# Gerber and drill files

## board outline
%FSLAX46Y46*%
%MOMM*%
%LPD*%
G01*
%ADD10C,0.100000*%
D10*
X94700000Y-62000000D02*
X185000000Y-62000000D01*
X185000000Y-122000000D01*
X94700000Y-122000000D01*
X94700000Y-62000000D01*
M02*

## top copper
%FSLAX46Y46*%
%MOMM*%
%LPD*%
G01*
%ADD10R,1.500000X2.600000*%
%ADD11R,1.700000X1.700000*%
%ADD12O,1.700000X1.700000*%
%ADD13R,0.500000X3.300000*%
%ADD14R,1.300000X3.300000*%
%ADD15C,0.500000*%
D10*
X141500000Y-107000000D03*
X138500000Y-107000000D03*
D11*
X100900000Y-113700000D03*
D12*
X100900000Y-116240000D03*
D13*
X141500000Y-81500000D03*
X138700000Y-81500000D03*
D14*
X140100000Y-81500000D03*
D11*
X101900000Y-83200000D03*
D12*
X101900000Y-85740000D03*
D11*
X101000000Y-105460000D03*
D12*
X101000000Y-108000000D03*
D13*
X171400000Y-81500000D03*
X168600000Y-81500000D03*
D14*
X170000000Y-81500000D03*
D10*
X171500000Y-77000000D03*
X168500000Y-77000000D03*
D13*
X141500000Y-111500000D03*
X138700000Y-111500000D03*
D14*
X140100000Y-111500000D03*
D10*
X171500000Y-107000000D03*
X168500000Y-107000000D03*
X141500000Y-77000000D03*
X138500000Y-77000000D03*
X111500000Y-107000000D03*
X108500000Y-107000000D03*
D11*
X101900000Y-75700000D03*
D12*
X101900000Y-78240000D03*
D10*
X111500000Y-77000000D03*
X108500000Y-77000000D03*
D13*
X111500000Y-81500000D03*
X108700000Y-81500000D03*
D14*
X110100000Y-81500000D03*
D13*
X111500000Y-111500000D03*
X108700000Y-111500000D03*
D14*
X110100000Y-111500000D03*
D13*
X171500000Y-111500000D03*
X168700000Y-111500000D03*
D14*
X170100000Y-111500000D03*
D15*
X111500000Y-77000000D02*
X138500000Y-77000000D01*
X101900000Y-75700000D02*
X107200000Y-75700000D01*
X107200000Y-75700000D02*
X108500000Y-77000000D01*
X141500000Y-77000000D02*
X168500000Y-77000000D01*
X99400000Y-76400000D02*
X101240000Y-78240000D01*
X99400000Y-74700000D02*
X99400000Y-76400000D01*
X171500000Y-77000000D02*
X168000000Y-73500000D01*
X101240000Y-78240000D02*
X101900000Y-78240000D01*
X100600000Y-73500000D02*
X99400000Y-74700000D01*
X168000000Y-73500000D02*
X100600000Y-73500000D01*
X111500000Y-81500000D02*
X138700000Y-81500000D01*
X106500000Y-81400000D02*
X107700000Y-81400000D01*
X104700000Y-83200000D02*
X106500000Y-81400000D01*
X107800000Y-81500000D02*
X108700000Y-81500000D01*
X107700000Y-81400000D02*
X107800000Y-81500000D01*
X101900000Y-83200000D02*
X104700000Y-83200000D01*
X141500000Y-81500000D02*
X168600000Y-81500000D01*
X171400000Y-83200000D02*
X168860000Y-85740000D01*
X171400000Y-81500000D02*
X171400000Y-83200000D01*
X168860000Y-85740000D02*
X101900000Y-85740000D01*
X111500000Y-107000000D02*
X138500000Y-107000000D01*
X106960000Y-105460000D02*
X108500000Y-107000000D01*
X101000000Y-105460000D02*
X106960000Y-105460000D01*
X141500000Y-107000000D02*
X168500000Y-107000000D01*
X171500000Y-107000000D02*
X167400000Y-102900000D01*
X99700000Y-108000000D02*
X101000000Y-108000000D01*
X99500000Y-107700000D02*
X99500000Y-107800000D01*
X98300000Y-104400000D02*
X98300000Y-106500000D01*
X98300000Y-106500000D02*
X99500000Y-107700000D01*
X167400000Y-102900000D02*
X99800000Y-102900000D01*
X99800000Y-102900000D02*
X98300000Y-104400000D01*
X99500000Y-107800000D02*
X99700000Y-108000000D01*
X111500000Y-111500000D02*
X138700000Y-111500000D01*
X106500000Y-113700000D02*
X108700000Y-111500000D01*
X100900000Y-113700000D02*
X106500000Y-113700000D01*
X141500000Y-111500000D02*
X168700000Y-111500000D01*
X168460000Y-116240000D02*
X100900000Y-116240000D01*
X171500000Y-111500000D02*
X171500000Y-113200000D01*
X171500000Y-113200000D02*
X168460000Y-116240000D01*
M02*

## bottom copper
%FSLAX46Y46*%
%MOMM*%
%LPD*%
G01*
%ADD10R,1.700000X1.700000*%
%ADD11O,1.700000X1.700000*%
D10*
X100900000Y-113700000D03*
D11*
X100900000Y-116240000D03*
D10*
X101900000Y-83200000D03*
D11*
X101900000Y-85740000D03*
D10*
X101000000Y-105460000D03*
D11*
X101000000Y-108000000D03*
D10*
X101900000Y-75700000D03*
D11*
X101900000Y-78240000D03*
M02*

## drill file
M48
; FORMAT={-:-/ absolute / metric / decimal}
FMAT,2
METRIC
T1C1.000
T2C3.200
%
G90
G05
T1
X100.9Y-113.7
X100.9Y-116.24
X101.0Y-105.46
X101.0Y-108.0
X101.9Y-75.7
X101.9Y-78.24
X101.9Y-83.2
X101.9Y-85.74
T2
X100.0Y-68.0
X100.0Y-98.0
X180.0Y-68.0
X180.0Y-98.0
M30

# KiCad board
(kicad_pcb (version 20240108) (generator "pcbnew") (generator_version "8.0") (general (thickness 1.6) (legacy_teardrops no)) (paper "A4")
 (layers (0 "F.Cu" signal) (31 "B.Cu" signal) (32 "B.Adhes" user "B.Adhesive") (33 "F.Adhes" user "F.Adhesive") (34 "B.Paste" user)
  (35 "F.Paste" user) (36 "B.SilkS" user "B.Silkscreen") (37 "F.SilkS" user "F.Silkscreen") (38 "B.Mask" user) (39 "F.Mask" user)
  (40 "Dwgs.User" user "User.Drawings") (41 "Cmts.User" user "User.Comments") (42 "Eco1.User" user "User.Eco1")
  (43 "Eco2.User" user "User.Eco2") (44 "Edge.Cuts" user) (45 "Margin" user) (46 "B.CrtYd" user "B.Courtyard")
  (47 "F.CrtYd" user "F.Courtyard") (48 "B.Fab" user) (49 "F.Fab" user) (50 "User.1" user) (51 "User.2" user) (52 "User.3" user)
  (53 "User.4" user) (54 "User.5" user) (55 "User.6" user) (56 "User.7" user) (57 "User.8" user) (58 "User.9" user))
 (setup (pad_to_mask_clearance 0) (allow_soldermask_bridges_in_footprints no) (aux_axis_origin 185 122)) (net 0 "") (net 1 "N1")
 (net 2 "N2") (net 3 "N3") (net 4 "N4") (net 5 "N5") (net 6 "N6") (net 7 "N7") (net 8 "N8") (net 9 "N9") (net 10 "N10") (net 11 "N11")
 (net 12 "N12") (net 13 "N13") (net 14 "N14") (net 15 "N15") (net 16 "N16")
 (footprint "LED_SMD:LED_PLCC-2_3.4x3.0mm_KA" (layer "F.Cu") (at 140 107 180)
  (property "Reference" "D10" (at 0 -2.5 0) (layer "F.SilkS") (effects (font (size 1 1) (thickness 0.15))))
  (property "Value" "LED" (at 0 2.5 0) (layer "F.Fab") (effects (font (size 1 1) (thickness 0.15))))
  (pad "1" smd rect (at -1.5 0 180) (size 1.5 2.6) (layers "F.Cu" "F.Paste" "F.Mask") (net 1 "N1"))
  (pad "2" smd rect (at 1.5 0 180) (size 1.5 2.6) (layers "F.Cu" "F.Paste" "F.Mask") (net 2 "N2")))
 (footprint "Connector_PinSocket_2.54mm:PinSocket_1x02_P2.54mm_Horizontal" (layer "F.Cu") (at 100.9 113.7)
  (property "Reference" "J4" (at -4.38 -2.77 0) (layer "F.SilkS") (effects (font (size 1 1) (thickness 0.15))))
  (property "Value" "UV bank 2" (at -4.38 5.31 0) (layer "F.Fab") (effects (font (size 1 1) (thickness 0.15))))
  (pad "1" thru_hole rect (at 0 0) (size 1.7 1.7) (drill 1) (layers "*.Cu" "*.Mask") (remove_unused_layers no) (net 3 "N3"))
  (pad "2" thru_hole oval (at 0 2.54) (size 1.7 1.7) (drill 1) (layers "*.Cu" "*.Mask") (remove_unused_layers no) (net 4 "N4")))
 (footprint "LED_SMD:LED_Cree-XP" (layer "F.Cu") (at 140.1 81.5 180)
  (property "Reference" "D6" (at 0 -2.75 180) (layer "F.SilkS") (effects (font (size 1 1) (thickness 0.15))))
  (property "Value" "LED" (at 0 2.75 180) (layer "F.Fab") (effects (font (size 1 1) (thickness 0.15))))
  (pad "" smd rect (at 0 -1 180) (size 1.01 0.75) (layers "F.Paste"))
  (pad "" smd rect (at 0 0 180) (size 1.01 0.75) (layers "F.Paste"))
  (pad "" smd rect (at 0 1 180) (size 1.01 0.75) (layers "F.Paste"))
  (pad "1" smd rect (at -1.4 0 180) (size 0.5 3.3) (layers "F.Cu" "F.Paste" "F.Mask") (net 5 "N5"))
  (pad "2" smd rect (at 1.4 0 180) (size 0.5 3.3) (layers "F.Cu" "F.Paste" "F.Mask") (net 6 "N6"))
  (pad "3" smd rect (at 0 0 180) (size 1.3 3.3) (layers "F.Cu" "F.Mask")))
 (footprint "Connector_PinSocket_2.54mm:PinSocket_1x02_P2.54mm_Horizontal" (layer "F.Cu") (at 101.9 83.2)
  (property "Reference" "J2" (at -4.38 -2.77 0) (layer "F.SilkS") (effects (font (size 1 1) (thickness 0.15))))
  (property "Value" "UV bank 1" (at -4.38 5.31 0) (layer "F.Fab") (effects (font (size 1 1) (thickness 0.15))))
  (pad "1" thru_hole rect (at 0 0) (size 1.7 1.7) (drill 1) (layers "*.Cu" "*.Mask") (remove_unused_layers no) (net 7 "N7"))
  (pad "2" thru_hole oval (at 0 2.54) (size 1.7 1.7) (drill 1) (layers "*.Cu" "*.Mask") (remove_unused_layers no) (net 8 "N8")))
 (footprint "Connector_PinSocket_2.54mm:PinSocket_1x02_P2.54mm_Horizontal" (layer "F.Cu") (at 101 105.46)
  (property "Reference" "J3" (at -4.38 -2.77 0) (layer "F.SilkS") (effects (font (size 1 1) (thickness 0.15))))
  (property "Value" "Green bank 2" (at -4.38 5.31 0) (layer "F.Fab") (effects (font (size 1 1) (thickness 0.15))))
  (pad "1" thru_hole rect (at 0 0) (size 1.7 1.7) (drill 1) (layers "*.Cu" "*.Mask") (remove_unused_layers no) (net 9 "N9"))
  (pad "2" thru_hole oval (at 0 2.54) (size 1.7 1.7) (drill 1) (layers "*.Cu" "*.Mask") (remove_unused_layers no) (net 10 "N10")))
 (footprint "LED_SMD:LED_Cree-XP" (layer "F.Cu") (at 170 81.5 180)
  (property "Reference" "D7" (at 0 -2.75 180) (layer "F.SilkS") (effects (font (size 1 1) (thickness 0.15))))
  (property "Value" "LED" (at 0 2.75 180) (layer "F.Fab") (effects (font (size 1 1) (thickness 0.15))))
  (pad "" smd rect (at 0 -1 180) (size 1.01 0.75) (layers "F.Paste"))
  (pad "" smd rect (at 0 0 180) (size 1.01 0.75) (layers "F.Paste"))
  (pad "" smd rect (at 0 1 180) (size 1.01 0.75) (layers "F.Paste"))
  (pad "1" smd rect (at -1.4 0 180) (size 0.5 3.3) (layers "F.Cu" "F.Paste" "F.Mask") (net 8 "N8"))
  (pad "2" smd rect (at 1.4 0 180) (size 0.5 3.3) (layers "F.Cu" "F.Paste" "F.Mask") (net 5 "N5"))
  (pad "3" smd rect (at 0 0 180) (size 1.3 3.3) (layers "F.Cu" "F.Mask")))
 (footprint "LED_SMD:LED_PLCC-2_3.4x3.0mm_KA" (layer "F.Cu") (at 170 77 180)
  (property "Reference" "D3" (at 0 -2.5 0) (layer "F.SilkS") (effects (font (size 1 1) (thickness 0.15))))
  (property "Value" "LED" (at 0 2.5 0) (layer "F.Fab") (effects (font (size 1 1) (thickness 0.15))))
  (pad "1" smd rect (at -1.5 0 180) (size 1.5 2.6) (layers "F.Cu" "F.Paste" "F.Mask") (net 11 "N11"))
  (pad "2" smd rect (at 1.5 0 180) (size 1.5 2.6) (layers "F.Cu" "F.Paste" "F.Mask") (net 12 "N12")))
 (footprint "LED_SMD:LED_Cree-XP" (layer "F.Cu") (at 140.1 111.5 180)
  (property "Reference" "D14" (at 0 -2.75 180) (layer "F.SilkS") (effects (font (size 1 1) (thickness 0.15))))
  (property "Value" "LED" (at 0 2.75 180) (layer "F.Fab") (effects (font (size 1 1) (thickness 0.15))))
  (pad "" smd rect (at 0 -1 180) (size 1.01 0.75) (layers "F.Paste"))
  (pad "" smd rect (at 0 0 180) (size 1.01 0.75) (layers "F.Paste"))
  (pad "" smd rect (at 0 1 180) (size 1.01 0.75) (layers "F.Paste"))
  (pad "1" smd rect (at -1.4 0 180) (size 0.5 3.3) (layers "F.Cu" "F.Paste" "F.Mask") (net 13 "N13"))
  (pad "2" smd rect (at 1.4 0 180) (size 0.5 3.3) (layers "F.Cu" "F.Paste" "F.Mask") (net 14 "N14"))
  (pad "3" smd rect (at 0 0 180) (size 1.3 3.3) (layers "F.Cu" "F.Mask")))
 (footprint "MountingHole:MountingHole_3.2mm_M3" (layer "F.Cu") (at 180 68)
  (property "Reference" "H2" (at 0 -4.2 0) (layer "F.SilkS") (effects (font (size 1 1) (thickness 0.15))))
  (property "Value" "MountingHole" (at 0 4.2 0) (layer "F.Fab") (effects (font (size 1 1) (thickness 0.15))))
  (pad "" np_thru_hole circle (at 0 0) (size 3.2 3.2) (drill 3.2) (layers "*.Cu" "*.Mask")))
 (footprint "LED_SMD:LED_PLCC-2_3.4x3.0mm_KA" (layer "F.Cu") (at 170 107 180)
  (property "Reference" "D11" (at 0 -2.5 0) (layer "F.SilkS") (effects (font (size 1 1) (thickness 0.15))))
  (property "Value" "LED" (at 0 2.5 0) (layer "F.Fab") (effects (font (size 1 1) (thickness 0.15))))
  (pad "1" smd rect (at -1.5 0 180) (size 1.5 2.6) (layers "F.Cu" "F.Paste" "F.Mask") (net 10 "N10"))
  (pad "2" smd rect (at 1.5 0 180) (size 1.5 2.6) (layers "F.Cu" "F.Paste" "F.Mask") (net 1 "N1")))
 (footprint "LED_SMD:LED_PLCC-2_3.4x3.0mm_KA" (layer "F.Cu") (at 140 77 180)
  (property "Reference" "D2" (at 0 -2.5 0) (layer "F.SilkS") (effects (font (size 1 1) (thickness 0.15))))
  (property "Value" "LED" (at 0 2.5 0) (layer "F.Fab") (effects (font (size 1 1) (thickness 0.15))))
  (pad "1" smd rect (at -1.5 0 180) (size 1.5 2.6) (layers "F.Cu" "F.Paste" "F.Mask") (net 12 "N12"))
  (pad "2" smd rect (at 1.5 0 180) (size 1.5 2.6) (layers "F.Cu" "F.Paste" "F.Mask") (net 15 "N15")))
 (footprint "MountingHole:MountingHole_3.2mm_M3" (layer "F.Cu") (at 100 98)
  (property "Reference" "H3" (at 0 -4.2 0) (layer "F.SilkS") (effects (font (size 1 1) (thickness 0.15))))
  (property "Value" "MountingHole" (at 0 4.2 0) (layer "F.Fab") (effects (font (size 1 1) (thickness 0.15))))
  (pad "" np_thru_hole circle (at 0 0) (size 3.2 3.2) (drill 3.2) (layers "*.Cu" "*.Mask")))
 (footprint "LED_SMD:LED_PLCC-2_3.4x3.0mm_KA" (layer "F.Cu") (at 110 107 180)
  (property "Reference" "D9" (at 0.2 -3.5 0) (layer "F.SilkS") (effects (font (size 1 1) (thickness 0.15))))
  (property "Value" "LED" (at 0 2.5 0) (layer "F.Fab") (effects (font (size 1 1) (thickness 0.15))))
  (pad "1" smd rect (at -1.5 0 180) (size 1.5 2.6) (layers "F.Cu" "F.Paste" "F.Mask") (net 2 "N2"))
  (pad "2" smd rect (at 1.5 0 180) (size 1.5 2.6) (layers "F.Cu" "F.Paste" "F.Mask") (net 9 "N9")))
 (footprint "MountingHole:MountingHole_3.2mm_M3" (layer "F.Cu") (at 180 98)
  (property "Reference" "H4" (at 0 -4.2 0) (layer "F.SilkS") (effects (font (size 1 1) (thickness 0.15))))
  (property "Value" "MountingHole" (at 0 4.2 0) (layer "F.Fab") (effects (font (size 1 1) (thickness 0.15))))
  (pad "" np_thru_hole circle (at 0 0) (size 3.2 3.2) (drill 3.2) (layers "*.Cu" "*.Mask")))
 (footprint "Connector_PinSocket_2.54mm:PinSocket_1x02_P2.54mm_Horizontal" (layer "F.Cu") (at 101.9 75.7)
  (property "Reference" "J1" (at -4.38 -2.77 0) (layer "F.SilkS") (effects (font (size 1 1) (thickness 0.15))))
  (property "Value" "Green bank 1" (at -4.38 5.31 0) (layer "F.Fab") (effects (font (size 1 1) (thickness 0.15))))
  (pad "1" thru_hole rect (at 0 0) (size 1.7 1.7) (drill 1) (layers "*.Cu" "*.Mask") (remove_unused_layers no) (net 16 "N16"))
  (pad "2" thru_hole oval (at 0 2.54) (size 1.7 1.7) (drill 1) (layers "*.Cu" "*.Mask") (remove_unused_layers no) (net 11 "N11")))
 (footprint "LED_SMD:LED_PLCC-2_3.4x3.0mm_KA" (layer "F.Cu") (at 110 77 180)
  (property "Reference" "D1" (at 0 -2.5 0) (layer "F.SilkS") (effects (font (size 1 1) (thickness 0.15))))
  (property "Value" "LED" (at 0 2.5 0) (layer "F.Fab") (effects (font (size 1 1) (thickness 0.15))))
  (pad "1" smd rect (at -1.5 0 180) (size 1.5 2.6) (layers "F.Cu" "F.Paste" "F.Mask") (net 15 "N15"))
  (pad "2" smd rect (at 1.5 0 180) (size 1.5 2.6) (layers "F.Cu" "F.Paste" "F.Mask") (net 16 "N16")))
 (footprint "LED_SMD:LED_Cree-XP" (layer "F.Cu") (at 110.1 81.5 180)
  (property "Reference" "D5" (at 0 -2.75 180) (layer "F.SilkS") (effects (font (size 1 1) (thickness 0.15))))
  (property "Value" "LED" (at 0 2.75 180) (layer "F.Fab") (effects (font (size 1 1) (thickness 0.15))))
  (pad "" smd rect (at 0 -1 180) (size 1.01 0.75) (layers "F.Paste"))
  (pad "" smd rect (at 0 0 180) (size 1.01 0.75) (layers "F.Paste"))
  (pad "" smd rect (at 0 1 180) (size 1.01 0.75) (layers "F.Paste"))
  (pad "1" smd rect (at -1.4 0 180) (size 0.5 3.3) (layers "F.Cu" "F.Paste" "F.Mask") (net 6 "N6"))
  (pad "2" smd rect (at 1.4 0 180) (size 0.5 3.3) (layers "F.Cu" "F.Paste" "F.Mask") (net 7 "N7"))
  (pad "3" smd rect (at 0 0 180) (size 1.3 3.3) (layers "F.Cu" "F.Mask")))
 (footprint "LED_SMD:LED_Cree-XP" (layer "F.Cu") (at 110.1 111.5 180)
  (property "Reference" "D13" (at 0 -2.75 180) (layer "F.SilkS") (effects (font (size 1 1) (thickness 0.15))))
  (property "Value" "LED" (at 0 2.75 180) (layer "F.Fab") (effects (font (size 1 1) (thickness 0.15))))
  (pad "" smd rect (at 0 -1 180) (size 1.01 0.75) (layers "F.Paste"))
  (pad "" smd rect (at 0 0 180) (size 1.01 0.75) (layers "F.Paste"))
  (pad "" smd rect (at 0 1 180) (size 1.01 0.75) (layers "F.Paste"))
  (pad "1" smd rect (at -1.4 0 180) (size 0.5 3.3) (layers "F.Cu" "F.Paste" "F.Mask") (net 14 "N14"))
  (pad "2" smd rect (at 1.4 0 180) (size 0.5 3.3) (layers "F.Cu" "F.Paste" "F.Mask") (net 3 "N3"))
  (pad "3" smd rect (at 0 0 180) (size 1.3 3.3) (layers "F.Cu" "F.Mask")))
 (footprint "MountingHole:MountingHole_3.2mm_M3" (layer "F.Cu") (at 100 68)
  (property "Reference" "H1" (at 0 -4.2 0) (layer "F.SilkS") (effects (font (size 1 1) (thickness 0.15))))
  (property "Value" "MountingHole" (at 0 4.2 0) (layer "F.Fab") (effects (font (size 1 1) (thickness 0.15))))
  (pad "" np_thru_hole circle (at 0 0) (size 3.2 3.2) (drill 3.2) (layers "*.Cu" "*.Mask")))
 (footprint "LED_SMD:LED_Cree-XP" (layer "F.Cu") (at 170.1 111.5 180)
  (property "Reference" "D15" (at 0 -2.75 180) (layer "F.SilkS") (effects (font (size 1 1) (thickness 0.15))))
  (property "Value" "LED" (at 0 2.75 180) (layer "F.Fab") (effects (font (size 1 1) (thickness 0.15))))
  (pad "" smd rect (at 0 -1 180) (size 1.01 0.75) (layers "F.Paste"))
  (pad "" smd rect (at 0 0 180) (size 1.01 0.75) (layers "F.Paste"))
  (pad "" smd rect (at 0 1 180) (size 1.01 0.75) (layers "F.Paste"))
  (pad "1" smd rect (at -1.4 0 180) (size 0.5 3.3) (layers "F.Cu" "F.Paste" "F.Mask") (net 4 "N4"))
  (pad "2" smd rect (at 1.4 0 180) (size 0.5 3.3) (layers "F.Cu" "F.Paste" "F.Mask") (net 13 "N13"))
  (pad "3" smd rect (at 0 0 180) (size 1.3 3.3) (layers "F.Cu" "F.Mask")))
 (gr_rect (start 94.7 62) (end 185 122) (stroke (width 0.1) (type default)) (fill none) (layer "Edge.Cuts"))
 (segment (start 111.5 77) (end 138.5 77) (width 0.5) (layer "F.Cu") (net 15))
 (segment (start 101.9 75.7) (end 107.2 75.7) (width 0.5) (layer "F.Cu") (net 16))
 (segment (start 107.2 75.7) (end 108.5 77) (width 0.5) (layer "F.Cu") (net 16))
 (segment (start 141.5 77) (end 168.5 77) (width 0.5) (layer "F.Cu") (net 12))
 (segment (start 99.4 76.4) (end 101.24 78.24) (width 0.5) (layer "F.Cu") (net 11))
 (segment (start 99.4 74.7) (end 99.4 76.4) (width 0.5) (layer "F.Cu") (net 11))
 (segment (start 171.5 77) (end 168 73.5) (width 0.5) (layer "F.Cu") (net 11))
 (segment (start 101.24 78.24) (end 101.9 78.24) (width 0.5) (layer "F.Cu") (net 11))
 (segment (start 100.6 73.5) (end 99.4 74.7) (width 0.5) (layer "F.Cu") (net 11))
 (segment (start 168 73.5) (end 100.6 73.5) (width 0.5) (layer "F.Cu") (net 11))
 (segment (start 111.5 81.5) (end 138.7 81.5) (width 0.5) (layer "F.Cu") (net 6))
 (segment (start 106.5 81.4) (end 107.7 81.4) (width 0.5) (layer "F.Cu") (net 7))
 (segment (start 104.7 83.2) (end 106.5 81.4) (width 0.5) (layer "F.Cu") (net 7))
 (segment (start 107.8 81.5) (end 108.7 81.5) (width 0.5) (layer "F.Cu") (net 7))
 (segment (start 107.7 81.4) (end 107.8 81.5) (width 0.5) (layer "F.Cu") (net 7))
 (segment (start 101.9 83.2) (end 104.7 83.2) (width 0.5) (layer "F.Cu") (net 7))
 (segment (start 141.5 81.5) (end 168.6 81.5) (width 0.5) (layer "F.Cu") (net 5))
 (segment (start 171.4 83.2) (end 168.86 85.74) (width 0.5) (layer "F.Cu") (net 8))
 (segment (start 171.4 81.5) (end 171.4 83.2) (width 0.5) (layer "F.Cu") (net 8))
 (segment (start 168.86 85.74) (end 101.9 85.74) (width 0.5) (layer "F.Cu") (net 8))
 (segment (start 111.5 107) (end 138.5 107) (width 0.5) (layer "F.Cu") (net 2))
 (segment (start 106.96 105.46) (end 108.5 107) (width 0.5) (layer "F.Cu") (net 9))
 (segment (start 101 105.46) (end 106.96 105.46) (width 0.5) (layer "F.Cu") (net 9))
 (segment (start 141.5 107) (end 168.5 107) (width 0.5) (layer "F.Cu") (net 1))
 (segment (start 171.5 107) (end 167.4 102.9) (width 0.5) (layer "F.Cu") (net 10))
 (segment (start 99.7 108) (end 101 108) (width 0.5) (layer "F.Cu") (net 10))
 (segment (start 99.5 107.7) (end 99.5 107.8) (width 0.5) (layer "F.Cu") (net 10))
 (segment (start 98.3 104.4) (end 98.3 106.5) (width 0.5) (layer "F.Cu") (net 10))
 (segment (start 98.3 106.5) (end 99.5 107.7) (width 0.5) (layer "F.Cu") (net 10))
 (segment (start 167.4 102.9) (end 99.8 102.9) (width 0.5) (layer "F.Cu") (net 10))
 (segment (start 99.8 102.9) (end 98.3 104.4) (width 0.5) (layer "F.Cu") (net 10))
 (segment (start 99.5 107.8) (end 99.7 108) (width 0.5) (layer "F.Cu") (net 10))
 (segment (start 111.5 111.5) (end 138.7 111.5) (width 0.5) (layer "F.Cu") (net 14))
 (segment (start 106.5 113.7) (end 108.7 111.5) (width 0.5) (layer "F.Cu") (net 3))
 (segment (start 100.9 113.7) (end 106.5 113.7) (width 0.5) (layer "F.Cu") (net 3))
 (segment (start 141.5 111.5) (end 168.7 111.5) (width 0.5) (layer "F.Cu") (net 13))
 (segment (start 168.46 116.24) (end 100.9 116.24) (width 0.5) (layer "F.Cu") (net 4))
 (segment (start 171.5 111.5) (end 171.5 113.2) (width 0.5) (layer "F.Cu") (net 4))
 (segment (start 171.5 113.2) (end 168.46 116.24) (width 0.5) (layer "F.Cu") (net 4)))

